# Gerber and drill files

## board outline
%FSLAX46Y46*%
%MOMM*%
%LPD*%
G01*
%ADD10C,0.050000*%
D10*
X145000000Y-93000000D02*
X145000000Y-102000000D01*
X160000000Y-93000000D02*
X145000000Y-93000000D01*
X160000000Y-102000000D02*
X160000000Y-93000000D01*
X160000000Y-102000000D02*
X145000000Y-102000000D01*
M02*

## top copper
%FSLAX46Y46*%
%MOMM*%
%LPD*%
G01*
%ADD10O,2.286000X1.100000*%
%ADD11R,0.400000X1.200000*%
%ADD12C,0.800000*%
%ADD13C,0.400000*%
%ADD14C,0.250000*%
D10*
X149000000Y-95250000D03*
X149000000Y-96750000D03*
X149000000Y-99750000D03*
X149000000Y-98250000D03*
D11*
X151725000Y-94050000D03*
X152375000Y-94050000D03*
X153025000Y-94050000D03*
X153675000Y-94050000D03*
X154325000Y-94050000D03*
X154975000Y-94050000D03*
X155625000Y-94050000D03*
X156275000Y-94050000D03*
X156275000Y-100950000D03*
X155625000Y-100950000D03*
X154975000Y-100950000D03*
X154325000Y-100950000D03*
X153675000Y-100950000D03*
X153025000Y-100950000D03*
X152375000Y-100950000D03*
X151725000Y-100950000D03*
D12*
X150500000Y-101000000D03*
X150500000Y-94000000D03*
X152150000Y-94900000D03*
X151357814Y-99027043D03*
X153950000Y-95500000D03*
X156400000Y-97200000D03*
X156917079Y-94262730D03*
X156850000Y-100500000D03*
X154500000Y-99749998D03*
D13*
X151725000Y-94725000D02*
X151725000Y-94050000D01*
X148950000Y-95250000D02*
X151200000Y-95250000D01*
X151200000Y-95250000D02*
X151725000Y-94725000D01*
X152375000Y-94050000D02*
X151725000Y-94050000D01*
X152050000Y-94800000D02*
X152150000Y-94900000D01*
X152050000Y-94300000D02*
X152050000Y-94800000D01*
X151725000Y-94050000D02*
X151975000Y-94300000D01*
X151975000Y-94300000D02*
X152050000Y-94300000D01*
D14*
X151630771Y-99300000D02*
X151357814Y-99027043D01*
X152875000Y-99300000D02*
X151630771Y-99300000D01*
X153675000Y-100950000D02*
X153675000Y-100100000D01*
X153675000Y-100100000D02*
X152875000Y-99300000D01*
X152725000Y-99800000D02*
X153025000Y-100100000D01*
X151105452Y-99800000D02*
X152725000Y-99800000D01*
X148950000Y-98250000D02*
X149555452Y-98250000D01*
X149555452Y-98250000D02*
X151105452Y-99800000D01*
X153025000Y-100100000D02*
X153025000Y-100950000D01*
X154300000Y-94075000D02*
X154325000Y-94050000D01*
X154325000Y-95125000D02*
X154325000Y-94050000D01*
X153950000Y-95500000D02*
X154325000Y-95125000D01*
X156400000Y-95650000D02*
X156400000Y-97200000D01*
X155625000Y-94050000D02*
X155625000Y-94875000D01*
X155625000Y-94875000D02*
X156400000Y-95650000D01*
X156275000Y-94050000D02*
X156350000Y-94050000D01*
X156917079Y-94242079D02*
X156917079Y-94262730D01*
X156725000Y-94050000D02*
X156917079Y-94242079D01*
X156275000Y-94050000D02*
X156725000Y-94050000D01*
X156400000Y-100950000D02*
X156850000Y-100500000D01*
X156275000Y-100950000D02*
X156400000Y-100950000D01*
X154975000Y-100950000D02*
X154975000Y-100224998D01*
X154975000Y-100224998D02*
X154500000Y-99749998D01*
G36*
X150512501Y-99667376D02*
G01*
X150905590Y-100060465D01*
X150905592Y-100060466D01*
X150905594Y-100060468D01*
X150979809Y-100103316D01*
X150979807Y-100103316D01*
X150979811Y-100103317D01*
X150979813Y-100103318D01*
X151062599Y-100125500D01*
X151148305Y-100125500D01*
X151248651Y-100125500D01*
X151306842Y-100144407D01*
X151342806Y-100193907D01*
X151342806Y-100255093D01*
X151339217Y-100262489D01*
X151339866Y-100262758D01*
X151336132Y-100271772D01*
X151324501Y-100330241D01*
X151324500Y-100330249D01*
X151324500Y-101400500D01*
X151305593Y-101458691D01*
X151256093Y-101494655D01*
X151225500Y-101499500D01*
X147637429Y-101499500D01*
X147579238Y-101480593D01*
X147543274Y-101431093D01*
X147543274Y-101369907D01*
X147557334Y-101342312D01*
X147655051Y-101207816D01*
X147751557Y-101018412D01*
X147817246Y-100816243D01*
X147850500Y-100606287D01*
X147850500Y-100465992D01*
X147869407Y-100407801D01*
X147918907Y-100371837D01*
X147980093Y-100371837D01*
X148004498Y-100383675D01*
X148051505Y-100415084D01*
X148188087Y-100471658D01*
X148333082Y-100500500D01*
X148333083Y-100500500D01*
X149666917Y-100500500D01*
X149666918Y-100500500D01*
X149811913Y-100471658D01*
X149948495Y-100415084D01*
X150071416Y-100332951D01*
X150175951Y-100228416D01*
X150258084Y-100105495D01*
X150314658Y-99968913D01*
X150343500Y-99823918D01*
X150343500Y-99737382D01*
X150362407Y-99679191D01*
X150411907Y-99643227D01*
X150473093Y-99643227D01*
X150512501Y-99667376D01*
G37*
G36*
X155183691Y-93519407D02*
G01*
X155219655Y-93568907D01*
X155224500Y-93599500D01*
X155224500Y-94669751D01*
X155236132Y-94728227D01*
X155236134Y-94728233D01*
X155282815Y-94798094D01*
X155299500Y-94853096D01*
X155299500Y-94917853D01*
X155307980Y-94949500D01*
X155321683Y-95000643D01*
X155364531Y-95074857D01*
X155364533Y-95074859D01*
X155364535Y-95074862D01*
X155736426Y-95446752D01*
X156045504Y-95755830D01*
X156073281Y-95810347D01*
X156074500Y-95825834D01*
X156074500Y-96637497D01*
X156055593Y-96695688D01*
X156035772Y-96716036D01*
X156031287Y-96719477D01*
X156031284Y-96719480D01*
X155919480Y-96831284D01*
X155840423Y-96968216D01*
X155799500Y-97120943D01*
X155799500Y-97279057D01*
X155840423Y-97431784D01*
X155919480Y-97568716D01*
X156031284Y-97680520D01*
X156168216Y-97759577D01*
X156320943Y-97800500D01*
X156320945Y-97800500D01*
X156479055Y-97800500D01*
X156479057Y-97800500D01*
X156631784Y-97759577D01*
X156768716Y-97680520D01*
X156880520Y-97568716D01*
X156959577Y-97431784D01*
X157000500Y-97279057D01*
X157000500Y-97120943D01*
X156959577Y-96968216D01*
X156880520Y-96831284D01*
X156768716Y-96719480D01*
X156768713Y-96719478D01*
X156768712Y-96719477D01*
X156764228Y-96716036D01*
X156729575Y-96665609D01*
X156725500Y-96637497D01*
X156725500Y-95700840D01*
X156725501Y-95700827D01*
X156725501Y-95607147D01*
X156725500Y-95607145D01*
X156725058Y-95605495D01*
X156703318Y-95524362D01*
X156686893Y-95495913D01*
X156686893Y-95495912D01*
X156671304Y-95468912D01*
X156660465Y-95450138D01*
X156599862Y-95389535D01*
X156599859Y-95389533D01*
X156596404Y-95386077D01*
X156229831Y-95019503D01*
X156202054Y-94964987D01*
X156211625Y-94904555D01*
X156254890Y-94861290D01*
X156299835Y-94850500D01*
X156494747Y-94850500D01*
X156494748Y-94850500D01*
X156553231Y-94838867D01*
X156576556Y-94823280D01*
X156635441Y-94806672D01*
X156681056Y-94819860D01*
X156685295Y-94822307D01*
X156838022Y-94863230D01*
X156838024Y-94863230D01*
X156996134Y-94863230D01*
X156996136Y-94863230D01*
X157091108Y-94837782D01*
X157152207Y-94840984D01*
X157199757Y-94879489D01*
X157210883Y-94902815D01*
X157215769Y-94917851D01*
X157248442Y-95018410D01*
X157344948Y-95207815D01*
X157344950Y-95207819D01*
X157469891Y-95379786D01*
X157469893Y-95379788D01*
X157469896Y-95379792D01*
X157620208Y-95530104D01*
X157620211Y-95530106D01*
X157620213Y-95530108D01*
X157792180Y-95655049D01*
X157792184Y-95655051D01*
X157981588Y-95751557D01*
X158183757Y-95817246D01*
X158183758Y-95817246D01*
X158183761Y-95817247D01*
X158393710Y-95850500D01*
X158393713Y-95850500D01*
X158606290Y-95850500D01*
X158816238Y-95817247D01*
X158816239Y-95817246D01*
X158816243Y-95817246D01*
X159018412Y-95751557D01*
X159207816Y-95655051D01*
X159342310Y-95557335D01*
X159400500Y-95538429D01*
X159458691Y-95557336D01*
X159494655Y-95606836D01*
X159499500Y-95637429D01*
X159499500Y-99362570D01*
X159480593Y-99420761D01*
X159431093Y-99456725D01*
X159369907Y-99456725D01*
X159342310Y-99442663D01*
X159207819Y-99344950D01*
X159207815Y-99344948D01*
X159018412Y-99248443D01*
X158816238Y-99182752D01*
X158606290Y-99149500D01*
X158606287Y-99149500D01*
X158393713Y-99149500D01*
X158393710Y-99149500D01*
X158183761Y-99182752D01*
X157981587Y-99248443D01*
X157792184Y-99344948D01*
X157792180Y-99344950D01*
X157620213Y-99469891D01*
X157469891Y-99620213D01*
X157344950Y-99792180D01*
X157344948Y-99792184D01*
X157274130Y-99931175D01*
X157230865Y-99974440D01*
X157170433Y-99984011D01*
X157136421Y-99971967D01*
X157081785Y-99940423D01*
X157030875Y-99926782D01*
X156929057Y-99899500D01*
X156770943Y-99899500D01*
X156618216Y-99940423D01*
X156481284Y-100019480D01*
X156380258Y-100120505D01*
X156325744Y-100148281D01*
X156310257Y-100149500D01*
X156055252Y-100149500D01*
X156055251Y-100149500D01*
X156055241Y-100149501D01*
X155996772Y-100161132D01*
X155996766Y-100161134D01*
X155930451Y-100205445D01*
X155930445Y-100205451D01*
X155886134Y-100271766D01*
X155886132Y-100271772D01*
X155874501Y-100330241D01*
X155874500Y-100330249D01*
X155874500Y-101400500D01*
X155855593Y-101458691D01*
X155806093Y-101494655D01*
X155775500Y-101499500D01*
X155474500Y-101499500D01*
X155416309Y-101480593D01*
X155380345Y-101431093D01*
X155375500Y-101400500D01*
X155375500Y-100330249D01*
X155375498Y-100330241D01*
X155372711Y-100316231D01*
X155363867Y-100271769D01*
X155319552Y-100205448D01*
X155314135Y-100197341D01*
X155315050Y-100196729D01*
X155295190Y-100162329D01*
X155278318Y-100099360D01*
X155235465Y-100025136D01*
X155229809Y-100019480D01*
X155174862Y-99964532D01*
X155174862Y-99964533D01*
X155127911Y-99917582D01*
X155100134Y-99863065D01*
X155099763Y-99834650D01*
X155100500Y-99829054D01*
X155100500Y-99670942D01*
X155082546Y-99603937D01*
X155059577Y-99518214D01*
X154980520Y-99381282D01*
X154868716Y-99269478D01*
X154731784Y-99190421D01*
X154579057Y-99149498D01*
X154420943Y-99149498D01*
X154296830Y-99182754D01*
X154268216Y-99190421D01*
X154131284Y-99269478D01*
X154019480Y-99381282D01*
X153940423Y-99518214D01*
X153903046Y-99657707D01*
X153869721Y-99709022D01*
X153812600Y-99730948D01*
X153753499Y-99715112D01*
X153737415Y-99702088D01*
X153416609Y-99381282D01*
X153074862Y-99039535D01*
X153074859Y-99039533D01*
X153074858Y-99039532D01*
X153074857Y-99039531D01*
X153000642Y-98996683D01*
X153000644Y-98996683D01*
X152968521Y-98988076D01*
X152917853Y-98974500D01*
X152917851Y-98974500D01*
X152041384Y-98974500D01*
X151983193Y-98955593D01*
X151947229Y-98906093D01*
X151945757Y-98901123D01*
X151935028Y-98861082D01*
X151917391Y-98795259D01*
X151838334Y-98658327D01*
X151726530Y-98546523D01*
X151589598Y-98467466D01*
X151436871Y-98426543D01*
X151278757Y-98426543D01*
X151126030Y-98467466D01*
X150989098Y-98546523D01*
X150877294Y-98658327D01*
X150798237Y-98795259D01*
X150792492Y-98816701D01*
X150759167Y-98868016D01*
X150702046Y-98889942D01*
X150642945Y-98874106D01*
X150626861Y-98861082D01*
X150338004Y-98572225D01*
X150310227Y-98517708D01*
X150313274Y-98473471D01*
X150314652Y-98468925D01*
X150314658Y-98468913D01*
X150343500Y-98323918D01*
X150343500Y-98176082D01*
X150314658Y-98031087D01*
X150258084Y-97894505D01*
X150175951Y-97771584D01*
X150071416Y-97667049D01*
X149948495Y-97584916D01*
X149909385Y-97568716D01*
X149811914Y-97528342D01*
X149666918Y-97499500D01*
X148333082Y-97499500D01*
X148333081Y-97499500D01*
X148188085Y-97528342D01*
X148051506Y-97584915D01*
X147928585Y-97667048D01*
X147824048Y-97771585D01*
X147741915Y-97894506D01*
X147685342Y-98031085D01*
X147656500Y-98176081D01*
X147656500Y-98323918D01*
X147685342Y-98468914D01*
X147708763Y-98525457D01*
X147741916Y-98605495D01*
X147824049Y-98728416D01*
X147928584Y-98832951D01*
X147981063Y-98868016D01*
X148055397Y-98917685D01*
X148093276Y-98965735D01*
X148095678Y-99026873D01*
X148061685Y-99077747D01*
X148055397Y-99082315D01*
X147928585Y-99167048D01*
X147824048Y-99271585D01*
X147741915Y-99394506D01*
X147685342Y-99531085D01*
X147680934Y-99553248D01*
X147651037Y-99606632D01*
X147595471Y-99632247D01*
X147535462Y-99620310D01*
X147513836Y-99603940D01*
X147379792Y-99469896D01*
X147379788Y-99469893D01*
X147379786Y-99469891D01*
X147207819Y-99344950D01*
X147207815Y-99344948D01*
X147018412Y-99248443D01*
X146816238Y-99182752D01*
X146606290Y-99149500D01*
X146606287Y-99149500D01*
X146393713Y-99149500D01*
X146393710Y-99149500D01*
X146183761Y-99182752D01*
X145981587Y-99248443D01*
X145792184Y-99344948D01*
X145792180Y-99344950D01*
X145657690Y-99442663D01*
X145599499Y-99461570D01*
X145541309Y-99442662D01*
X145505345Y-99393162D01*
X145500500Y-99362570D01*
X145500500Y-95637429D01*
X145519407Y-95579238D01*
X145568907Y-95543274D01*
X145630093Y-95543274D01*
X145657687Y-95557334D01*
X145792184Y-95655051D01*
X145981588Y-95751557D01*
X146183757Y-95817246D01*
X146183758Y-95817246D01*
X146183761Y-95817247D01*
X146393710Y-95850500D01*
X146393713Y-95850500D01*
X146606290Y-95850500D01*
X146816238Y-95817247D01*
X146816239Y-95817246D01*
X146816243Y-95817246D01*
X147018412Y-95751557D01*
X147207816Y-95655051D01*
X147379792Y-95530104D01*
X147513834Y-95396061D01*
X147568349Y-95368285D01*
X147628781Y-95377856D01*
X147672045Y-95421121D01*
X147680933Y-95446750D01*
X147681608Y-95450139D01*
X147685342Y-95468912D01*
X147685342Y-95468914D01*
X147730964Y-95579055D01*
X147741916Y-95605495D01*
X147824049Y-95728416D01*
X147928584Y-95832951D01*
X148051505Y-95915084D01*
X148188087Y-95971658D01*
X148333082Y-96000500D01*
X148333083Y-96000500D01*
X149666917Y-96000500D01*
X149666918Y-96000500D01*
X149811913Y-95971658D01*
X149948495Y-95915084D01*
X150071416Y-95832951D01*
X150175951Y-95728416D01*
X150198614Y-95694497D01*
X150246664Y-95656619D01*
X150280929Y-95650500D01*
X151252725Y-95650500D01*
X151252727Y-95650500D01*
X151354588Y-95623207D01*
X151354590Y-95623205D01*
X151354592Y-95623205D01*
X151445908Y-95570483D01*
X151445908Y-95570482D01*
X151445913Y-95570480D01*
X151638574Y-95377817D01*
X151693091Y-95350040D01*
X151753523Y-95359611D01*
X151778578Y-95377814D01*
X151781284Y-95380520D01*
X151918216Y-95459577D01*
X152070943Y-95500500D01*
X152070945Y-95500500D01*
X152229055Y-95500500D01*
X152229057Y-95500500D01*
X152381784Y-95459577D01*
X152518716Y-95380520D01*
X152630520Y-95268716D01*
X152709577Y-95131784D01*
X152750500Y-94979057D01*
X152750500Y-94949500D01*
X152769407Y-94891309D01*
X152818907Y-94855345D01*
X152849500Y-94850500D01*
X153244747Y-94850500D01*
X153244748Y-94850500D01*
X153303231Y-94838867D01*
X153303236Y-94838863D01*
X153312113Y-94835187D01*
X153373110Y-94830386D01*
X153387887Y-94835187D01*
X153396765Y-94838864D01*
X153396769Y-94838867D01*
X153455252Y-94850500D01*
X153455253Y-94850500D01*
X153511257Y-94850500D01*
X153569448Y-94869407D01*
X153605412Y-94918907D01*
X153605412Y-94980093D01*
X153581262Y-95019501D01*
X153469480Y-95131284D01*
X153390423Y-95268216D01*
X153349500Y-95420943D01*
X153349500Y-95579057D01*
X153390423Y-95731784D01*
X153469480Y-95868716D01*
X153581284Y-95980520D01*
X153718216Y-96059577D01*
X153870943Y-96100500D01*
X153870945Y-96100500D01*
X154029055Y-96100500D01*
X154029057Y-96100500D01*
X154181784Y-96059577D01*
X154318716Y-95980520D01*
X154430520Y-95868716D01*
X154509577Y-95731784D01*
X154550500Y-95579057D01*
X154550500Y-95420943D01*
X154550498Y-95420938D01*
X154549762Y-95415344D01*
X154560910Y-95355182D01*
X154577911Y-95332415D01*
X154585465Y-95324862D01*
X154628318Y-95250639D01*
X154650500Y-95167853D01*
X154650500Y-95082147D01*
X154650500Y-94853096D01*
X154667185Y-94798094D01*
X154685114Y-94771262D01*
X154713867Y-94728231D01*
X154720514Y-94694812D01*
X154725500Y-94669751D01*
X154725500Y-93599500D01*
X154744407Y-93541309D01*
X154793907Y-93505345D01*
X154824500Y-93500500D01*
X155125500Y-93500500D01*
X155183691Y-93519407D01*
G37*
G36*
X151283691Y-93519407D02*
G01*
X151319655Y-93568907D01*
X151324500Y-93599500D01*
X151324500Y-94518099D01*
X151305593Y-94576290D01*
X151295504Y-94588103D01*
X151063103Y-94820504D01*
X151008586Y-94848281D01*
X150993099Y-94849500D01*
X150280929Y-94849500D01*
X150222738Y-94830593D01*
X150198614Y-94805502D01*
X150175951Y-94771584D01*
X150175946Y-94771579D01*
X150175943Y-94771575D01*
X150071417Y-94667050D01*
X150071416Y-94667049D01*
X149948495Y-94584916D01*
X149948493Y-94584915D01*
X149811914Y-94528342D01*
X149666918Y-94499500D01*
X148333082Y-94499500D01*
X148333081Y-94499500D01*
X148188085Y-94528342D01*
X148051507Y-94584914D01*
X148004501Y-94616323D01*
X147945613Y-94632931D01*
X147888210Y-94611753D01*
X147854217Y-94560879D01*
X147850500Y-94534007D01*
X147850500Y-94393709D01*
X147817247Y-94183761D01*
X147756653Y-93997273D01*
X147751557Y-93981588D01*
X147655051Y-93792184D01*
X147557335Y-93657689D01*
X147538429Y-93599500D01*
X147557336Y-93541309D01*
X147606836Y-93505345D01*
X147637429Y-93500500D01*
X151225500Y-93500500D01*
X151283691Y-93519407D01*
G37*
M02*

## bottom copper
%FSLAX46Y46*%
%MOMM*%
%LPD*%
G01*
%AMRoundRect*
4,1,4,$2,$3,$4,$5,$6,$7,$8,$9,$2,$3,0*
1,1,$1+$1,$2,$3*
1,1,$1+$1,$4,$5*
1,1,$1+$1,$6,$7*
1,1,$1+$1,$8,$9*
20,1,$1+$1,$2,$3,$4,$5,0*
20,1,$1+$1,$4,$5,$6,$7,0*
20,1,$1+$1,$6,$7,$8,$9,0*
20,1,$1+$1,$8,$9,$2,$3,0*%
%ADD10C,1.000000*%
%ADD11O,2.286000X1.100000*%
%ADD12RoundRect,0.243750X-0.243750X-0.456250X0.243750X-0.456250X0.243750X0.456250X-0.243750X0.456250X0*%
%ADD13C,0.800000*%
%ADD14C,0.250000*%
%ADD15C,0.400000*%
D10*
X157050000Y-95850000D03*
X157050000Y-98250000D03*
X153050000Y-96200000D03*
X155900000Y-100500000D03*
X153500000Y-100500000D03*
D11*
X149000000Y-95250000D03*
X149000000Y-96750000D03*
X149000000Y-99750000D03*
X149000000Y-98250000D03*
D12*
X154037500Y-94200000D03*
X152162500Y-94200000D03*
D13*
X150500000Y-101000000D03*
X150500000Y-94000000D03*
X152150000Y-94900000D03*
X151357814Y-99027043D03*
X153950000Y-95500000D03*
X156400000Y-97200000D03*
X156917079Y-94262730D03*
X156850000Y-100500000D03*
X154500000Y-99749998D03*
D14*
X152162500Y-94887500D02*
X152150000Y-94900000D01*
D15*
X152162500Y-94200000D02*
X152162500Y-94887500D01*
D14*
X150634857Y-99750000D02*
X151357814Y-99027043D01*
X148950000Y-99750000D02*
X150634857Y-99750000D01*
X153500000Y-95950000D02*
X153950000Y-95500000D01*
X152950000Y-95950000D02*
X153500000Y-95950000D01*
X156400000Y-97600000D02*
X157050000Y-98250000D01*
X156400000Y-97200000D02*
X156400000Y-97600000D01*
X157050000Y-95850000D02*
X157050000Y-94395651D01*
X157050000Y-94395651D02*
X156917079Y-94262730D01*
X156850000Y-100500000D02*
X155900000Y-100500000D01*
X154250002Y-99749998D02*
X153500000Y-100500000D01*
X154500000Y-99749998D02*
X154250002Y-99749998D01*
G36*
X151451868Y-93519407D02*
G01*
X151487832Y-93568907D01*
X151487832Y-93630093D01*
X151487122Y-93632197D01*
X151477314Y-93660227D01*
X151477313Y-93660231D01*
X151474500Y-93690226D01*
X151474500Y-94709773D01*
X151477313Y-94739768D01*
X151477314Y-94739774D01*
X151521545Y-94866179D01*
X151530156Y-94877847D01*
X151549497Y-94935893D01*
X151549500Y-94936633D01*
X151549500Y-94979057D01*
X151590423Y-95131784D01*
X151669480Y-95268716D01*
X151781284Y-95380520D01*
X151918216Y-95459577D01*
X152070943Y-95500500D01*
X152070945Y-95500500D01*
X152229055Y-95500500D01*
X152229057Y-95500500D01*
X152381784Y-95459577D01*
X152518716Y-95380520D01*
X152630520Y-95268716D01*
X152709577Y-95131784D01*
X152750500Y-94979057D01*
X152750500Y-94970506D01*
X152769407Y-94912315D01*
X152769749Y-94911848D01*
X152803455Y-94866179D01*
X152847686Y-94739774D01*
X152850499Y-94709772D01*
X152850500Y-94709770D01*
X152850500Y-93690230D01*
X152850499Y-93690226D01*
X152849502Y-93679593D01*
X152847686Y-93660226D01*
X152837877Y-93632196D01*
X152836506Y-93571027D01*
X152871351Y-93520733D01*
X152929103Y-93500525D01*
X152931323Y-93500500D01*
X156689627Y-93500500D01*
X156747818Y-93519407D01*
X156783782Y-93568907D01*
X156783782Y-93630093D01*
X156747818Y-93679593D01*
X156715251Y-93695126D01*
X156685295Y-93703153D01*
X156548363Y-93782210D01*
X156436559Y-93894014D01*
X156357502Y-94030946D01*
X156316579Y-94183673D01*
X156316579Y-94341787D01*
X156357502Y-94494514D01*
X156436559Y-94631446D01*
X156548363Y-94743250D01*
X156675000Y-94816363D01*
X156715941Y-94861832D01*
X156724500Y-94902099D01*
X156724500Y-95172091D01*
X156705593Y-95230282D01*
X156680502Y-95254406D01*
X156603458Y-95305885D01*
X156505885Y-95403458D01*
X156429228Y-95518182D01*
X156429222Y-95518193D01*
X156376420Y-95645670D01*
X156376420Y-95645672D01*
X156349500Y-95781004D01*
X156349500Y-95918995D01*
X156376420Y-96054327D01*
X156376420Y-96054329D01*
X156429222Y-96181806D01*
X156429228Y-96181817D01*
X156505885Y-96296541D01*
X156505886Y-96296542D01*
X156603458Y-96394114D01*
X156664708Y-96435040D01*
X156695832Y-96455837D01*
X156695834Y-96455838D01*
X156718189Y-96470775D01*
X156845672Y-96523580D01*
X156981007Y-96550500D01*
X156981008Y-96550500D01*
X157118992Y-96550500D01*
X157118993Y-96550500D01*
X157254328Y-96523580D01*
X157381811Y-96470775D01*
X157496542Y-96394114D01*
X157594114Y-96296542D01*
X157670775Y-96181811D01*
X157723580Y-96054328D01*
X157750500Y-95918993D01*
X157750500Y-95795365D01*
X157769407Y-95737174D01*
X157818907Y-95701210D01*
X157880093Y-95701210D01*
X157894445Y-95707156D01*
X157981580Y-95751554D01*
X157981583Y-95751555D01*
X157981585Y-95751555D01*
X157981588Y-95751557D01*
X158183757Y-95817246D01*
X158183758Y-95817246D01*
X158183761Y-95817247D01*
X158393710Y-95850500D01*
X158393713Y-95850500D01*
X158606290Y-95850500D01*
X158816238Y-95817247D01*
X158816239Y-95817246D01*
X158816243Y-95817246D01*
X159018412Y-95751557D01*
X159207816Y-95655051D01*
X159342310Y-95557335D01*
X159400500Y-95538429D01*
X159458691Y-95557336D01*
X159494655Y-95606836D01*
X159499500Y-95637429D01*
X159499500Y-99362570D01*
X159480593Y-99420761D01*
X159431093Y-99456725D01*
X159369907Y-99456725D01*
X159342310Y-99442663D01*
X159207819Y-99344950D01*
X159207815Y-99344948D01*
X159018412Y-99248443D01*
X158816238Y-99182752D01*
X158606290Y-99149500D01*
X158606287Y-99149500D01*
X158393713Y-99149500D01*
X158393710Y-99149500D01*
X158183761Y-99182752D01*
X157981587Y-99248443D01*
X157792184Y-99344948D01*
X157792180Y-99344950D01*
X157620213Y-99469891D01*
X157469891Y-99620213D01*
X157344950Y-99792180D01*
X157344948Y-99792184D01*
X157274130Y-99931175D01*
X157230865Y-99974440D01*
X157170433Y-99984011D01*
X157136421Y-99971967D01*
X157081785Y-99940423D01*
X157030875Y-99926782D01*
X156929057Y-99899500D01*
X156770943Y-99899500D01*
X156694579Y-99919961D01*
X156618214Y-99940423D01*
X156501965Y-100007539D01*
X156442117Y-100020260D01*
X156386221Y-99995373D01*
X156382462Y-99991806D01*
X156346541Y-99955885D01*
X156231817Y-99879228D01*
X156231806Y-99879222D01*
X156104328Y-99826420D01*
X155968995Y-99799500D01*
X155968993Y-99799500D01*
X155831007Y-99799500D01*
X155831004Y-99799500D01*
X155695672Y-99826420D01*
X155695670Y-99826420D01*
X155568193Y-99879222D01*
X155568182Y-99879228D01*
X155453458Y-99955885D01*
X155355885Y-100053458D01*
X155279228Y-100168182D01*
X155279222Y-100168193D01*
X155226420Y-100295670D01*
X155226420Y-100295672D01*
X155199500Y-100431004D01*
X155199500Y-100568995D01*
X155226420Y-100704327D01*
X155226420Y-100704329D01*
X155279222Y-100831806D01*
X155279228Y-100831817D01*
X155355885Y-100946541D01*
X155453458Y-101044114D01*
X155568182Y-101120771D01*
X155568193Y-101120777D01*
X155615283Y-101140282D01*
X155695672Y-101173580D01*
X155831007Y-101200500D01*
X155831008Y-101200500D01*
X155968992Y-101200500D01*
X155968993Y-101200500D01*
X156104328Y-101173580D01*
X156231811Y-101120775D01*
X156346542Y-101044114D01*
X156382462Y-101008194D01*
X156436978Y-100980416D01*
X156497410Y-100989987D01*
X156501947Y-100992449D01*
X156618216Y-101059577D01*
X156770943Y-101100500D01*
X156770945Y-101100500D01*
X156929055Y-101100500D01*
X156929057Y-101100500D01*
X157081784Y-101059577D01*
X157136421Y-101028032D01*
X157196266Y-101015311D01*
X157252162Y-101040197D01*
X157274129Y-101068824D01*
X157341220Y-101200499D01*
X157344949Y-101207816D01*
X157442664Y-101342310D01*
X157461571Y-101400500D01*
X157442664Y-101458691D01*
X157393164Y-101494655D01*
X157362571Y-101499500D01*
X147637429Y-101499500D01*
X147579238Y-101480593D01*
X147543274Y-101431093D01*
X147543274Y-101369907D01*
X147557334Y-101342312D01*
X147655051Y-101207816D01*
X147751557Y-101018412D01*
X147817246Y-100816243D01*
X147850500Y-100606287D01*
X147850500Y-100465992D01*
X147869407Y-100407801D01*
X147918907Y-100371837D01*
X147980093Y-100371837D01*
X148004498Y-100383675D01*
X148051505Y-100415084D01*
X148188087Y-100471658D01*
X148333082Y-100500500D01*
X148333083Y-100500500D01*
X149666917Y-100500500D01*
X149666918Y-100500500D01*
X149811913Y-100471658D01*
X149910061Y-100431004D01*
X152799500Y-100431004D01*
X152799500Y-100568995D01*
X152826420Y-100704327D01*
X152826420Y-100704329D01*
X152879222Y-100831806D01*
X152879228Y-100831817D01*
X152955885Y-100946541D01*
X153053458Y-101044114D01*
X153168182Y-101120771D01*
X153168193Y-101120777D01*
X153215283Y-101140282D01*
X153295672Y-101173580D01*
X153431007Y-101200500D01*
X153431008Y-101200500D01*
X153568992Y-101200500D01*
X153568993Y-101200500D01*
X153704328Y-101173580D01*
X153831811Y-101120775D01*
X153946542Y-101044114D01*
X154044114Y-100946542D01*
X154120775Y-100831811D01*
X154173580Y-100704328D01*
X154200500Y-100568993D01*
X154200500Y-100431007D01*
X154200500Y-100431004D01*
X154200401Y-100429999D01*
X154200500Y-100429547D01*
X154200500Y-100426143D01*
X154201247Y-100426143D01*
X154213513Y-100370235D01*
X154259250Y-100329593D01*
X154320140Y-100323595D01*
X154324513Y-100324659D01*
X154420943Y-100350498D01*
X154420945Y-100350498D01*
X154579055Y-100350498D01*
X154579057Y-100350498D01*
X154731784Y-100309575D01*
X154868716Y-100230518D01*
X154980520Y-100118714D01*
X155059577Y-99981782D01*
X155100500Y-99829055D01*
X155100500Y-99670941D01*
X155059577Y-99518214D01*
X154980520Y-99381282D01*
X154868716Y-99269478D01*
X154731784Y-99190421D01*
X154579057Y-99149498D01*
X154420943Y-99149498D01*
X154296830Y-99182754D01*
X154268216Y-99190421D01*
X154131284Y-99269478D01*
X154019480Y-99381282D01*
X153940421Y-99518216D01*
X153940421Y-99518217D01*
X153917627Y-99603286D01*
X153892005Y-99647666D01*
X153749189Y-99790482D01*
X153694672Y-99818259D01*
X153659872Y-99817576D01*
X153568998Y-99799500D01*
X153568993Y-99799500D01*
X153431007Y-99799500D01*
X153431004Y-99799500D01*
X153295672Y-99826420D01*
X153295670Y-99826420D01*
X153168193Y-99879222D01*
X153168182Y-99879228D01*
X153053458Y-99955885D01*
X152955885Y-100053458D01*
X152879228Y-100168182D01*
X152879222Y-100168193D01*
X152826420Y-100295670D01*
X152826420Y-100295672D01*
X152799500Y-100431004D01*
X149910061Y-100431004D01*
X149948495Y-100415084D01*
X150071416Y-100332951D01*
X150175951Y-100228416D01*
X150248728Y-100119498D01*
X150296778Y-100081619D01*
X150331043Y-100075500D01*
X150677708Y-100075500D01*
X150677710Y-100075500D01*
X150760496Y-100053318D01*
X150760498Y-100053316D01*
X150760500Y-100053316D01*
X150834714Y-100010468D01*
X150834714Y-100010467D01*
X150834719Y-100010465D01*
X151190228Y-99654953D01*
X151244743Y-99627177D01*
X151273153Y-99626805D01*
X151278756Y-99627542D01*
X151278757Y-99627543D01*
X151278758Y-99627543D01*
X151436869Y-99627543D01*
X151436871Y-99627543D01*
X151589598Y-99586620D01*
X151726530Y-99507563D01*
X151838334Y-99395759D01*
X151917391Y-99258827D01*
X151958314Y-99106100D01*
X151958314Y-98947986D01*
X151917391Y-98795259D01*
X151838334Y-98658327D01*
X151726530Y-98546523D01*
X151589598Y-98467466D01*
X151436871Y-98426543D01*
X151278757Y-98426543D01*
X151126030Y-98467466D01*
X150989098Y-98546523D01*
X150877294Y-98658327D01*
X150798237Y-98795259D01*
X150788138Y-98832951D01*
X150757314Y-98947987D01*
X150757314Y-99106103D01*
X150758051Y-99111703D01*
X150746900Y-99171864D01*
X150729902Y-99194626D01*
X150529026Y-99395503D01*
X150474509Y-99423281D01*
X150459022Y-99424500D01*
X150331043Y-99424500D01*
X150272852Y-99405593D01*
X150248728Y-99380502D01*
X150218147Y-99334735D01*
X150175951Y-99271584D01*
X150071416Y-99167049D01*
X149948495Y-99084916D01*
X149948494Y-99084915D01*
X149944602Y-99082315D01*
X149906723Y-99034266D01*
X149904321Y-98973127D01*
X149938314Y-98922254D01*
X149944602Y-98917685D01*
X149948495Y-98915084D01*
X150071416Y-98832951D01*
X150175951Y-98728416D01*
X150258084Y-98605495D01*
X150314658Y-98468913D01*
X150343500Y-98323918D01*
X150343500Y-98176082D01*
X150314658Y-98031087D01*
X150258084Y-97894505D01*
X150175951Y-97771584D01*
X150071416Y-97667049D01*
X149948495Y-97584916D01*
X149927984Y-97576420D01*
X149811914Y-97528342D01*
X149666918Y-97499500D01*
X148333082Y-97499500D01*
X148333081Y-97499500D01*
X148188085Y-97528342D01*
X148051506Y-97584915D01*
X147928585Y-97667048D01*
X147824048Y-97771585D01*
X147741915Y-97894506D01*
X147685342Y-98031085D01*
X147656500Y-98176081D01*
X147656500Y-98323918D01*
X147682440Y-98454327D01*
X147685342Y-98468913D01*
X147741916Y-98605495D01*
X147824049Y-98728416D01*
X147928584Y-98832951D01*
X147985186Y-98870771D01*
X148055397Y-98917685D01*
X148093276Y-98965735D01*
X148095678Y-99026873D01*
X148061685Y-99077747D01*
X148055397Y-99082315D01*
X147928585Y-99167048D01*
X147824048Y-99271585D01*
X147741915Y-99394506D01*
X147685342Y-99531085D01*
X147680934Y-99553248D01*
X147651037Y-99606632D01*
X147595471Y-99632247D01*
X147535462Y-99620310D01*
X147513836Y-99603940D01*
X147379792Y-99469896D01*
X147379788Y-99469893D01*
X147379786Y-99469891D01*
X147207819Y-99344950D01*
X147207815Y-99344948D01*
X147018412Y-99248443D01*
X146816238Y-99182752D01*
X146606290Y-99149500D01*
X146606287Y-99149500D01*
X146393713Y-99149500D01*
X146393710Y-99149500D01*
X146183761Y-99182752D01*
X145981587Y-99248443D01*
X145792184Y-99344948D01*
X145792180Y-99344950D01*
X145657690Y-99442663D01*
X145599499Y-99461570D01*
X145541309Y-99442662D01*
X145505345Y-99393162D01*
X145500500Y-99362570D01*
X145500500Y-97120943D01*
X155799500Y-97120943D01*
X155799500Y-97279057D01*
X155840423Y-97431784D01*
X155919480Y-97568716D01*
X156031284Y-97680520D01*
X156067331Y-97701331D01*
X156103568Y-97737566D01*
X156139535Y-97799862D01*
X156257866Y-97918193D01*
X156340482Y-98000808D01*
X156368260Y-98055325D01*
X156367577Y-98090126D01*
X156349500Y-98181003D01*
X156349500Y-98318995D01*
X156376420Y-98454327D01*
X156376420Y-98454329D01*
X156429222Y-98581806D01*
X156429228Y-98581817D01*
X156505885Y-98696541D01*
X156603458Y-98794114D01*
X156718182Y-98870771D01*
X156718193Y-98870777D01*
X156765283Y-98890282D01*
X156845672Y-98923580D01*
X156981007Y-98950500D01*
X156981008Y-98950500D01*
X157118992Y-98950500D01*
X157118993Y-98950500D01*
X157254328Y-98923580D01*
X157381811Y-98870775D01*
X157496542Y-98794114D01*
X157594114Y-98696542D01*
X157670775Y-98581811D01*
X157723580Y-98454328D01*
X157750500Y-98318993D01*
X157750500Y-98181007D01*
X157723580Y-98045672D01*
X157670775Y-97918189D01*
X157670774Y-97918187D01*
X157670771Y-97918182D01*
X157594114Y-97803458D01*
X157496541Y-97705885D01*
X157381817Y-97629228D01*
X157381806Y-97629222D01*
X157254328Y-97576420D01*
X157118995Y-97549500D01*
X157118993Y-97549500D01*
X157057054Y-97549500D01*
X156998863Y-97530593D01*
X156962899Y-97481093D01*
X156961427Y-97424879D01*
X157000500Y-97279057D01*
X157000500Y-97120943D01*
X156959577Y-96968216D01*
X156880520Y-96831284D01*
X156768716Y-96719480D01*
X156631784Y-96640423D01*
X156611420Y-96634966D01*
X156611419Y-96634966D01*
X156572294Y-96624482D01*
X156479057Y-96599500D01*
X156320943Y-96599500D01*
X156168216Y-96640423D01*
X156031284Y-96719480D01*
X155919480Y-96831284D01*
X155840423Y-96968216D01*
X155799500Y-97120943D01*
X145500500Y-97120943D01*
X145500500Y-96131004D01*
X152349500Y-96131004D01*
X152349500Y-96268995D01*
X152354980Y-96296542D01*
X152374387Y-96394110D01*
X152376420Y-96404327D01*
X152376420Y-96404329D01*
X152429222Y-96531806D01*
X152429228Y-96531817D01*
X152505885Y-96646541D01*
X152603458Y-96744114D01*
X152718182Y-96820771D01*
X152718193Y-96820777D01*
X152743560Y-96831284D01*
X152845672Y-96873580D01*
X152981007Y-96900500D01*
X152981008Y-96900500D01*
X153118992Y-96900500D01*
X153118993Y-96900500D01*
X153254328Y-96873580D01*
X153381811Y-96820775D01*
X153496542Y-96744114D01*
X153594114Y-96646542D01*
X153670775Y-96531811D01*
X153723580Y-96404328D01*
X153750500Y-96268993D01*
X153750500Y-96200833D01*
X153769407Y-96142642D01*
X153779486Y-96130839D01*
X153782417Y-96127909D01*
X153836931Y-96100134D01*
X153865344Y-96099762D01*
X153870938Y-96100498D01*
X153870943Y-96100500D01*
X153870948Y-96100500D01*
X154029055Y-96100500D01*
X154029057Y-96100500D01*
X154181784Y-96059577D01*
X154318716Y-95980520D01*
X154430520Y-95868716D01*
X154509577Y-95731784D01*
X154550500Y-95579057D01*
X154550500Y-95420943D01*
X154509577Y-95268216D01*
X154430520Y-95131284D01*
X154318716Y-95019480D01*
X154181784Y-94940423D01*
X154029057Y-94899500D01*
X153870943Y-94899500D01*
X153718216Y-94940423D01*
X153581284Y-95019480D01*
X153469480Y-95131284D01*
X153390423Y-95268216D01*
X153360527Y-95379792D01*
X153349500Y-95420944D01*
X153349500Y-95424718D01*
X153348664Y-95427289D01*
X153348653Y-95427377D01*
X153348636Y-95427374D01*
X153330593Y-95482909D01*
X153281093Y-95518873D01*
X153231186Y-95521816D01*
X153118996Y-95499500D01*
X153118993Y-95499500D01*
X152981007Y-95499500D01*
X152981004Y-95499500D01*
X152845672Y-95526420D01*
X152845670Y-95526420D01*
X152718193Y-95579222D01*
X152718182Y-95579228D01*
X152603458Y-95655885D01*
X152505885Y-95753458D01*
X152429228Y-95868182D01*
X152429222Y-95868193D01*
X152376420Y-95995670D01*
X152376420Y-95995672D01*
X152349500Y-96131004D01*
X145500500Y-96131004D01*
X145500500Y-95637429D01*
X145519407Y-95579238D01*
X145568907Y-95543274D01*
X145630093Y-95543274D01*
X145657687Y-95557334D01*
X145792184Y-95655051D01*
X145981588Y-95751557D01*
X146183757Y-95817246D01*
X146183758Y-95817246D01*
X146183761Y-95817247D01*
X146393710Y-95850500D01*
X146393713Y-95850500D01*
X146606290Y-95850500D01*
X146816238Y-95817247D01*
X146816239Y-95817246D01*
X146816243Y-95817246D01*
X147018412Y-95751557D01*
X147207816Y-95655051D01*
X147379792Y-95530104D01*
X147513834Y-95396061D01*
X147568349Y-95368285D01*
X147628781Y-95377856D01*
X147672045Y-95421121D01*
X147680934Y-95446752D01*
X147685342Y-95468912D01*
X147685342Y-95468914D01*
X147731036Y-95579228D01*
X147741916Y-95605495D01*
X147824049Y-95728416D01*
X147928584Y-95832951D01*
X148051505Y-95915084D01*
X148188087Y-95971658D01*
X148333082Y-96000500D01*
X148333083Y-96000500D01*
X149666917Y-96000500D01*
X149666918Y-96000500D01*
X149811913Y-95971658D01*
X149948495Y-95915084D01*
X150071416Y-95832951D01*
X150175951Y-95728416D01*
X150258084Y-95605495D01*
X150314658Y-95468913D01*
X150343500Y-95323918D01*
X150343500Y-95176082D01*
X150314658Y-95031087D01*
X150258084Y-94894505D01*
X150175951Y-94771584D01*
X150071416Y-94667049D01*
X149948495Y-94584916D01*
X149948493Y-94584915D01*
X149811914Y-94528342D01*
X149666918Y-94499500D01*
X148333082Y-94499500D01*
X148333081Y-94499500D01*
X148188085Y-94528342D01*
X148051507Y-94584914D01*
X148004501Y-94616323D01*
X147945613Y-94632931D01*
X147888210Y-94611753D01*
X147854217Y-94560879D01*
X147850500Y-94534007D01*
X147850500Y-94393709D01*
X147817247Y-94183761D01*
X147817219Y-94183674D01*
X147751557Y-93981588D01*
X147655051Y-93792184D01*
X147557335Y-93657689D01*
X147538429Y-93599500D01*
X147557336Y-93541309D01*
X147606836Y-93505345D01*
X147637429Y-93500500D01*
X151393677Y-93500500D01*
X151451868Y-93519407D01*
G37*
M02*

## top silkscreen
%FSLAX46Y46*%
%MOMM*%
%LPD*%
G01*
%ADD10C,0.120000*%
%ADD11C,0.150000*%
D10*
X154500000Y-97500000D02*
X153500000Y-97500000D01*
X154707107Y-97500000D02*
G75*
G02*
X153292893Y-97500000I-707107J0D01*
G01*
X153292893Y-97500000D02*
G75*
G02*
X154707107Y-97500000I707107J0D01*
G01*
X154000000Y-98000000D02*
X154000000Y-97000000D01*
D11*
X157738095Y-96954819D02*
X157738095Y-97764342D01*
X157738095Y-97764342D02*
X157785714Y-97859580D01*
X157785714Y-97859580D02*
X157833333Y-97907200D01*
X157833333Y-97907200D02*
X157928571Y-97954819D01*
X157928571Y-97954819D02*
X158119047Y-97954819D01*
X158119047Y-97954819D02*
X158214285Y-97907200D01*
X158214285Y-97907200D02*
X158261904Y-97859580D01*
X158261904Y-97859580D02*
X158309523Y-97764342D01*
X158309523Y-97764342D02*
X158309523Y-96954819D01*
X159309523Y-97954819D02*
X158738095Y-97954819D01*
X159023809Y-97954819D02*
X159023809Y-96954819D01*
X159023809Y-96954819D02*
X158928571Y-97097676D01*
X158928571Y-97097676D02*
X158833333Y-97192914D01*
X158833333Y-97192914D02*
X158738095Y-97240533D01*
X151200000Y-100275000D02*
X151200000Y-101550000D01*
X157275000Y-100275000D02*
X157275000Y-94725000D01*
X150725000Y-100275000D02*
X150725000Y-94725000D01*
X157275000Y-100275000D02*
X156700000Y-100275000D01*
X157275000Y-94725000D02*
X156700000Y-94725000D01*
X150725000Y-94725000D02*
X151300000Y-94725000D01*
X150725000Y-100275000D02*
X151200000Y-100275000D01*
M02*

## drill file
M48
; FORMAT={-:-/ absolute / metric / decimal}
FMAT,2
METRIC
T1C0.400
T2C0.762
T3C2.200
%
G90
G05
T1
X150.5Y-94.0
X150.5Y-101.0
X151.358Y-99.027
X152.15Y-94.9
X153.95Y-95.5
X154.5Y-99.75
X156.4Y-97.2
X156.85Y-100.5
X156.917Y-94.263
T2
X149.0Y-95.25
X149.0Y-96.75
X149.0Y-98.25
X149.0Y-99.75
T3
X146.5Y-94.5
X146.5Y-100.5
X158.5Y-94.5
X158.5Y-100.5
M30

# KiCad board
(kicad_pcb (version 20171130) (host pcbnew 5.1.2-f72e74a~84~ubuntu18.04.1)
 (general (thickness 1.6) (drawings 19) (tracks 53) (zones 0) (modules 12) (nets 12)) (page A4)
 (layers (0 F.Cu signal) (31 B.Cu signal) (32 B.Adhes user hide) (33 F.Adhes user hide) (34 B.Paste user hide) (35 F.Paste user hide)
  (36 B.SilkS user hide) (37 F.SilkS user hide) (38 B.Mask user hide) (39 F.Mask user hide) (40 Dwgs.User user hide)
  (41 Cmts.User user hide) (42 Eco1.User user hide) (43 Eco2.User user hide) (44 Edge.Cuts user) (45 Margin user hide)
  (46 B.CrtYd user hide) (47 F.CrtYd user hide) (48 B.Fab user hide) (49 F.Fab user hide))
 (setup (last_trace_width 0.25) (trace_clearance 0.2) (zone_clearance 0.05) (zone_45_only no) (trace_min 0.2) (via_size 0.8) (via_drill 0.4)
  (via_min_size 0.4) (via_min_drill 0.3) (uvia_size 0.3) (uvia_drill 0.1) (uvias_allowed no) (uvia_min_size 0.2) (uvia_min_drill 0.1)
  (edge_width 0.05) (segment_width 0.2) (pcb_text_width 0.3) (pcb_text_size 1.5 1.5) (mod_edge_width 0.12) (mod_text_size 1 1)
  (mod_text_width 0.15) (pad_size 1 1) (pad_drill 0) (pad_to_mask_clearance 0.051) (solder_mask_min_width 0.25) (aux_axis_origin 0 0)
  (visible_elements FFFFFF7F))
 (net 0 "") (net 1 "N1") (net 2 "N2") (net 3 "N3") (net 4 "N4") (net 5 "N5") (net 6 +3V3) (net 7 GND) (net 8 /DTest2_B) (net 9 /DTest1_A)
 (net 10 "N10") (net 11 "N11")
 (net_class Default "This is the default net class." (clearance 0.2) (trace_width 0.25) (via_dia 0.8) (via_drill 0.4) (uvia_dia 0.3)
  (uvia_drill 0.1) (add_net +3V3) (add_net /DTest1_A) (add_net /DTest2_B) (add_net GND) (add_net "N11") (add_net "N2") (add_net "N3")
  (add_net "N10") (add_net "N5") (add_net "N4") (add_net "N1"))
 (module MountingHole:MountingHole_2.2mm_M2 (layer F.Cu) (at 146.5 100.5)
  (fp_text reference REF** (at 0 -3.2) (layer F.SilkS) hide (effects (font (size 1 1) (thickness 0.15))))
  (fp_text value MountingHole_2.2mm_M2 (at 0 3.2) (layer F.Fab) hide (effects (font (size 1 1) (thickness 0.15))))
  (pad 1 np_thru_hole circle (at 0 0) (size 2.2 2.2) (drill 2.2) (layers *.Cu *.Mask)))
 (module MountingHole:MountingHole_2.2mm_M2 (layer F.Cu) (at 146.5 94.5)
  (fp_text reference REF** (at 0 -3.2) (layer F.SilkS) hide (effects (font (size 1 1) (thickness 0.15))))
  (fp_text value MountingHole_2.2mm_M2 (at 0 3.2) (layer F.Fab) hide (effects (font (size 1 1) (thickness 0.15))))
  (pad 1 np_thru_hole circle (at 0 0) (size 2.2 2.2) (drill 2.2) (layers *.Cu *.Mask)))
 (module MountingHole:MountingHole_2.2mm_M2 (layer F.Cu) (at 158.5 94.5)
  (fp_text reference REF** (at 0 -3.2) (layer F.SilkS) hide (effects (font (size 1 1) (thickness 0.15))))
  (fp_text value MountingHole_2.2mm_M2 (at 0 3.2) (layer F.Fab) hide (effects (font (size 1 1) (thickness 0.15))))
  (pad 1 np_thru_hole circle (at 0 0) (size 2.2 2.2) (drill 2.2) (layers *.Cu *.Mask)))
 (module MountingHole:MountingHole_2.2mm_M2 (layer F.Cu) (at 158.5 100.5)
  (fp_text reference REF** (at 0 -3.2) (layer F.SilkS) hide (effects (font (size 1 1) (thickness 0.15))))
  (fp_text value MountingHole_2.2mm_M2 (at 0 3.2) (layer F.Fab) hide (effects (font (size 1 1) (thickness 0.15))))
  (pad 1 np_thru_hole circle (at 0 0) (size 2.2 2.2) (drill 2.2) (layers *.Cu *.Mask)))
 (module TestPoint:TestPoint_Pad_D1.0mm (layer B.Cu) (at 157.05 95.85)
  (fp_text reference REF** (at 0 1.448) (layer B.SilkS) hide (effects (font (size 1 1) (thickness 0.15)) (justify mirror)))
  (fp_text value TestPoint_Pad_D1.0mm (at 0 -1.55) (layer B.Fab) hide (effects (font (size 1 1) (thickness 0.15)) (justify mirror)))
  (pad 1 smd circle (at 0 0) (size 1 1) (layers B.Cu B.Mask) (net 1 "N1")))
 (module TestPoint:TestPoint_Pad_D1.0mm (layer B.Cu) (at 157.05 98.25)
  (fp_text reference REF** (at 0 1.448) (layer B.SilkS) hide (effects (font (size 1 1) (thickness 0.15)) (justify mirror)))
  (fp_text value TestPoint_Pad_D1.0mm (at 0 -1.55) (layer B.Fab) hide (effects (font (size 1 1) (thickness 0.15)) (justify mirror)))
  (pad 1 smd circle (at 0 0) (size 1 1) (layers B.Cu B.Mask) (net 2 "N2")))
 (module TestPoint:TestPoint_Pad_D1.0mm (layer B.Cu) (at 153.05 96.2)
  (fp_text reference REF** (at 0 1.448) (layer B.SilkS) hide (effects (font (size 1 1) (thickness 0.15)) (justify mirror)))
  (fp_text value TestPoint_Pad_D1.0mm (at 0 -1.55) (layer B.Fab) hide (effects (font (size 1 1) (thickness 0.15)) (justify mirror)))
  (pad 1 smd circle (at 0 0) (size 1 1) (layers B.Cu B.Mask) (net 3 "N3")))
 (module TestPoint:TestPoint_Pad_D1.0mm (layer B.Cu) (at 155.9 100.5)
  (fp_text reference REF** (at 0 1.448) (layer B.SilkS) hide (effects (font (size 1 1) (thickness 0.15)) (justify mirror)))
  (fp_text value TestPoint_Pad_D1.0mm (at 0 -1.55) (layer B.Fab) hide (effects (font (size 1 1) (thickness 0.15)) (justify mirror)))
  (pad 1 smd circle (at 0 0) (size 1 1) (layers B.Cu B.Mask) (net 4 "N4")))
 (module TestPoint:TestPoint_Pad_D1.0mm (layer B.Cu) (at 153.5 100.5)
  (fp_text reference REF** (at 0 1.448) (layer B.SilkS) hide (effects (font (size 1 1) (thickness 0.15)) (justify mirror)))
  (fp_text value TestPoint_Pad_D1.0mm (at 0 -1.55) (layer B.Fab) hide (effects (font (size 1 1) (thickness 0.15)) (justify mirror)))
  (pad 1 smd circle (at 0 0) (size 1 1) (layers B.Cu B.Mask) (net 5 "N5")))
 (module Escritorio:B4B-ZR (layer B.Cu) (at 149.45 97.5 270)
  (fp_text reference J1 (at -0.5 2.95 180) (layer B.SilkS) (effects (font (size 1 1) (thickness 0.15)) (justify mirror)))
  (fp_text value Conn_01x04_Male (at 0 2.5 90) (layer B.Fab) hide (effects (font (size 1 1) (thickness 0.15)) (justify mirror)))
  (pad 1 thru_hole oval (at -2.25 0.45 270) (size 1.1 2.286) (drill 0.762) (layers *.Cu *.Mask) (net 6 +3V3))
  (pad 2 thru_hole oval (at -0.75 0.45 270) (size 1.1 2.286) (drill 0.762) (layers *.Cu *.Mask) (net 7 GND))
  (pad 4 thru_hole oval (at 2.25 0.45 270) (size 1.1 2.286) (drill 0.762) (layers *.Cu *.Mask) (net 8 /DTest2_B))
  (pad 3 thru_hole oval (at 0.75 0.45 270) (size 1.1 2.286) (drill 0.762) (layers *.Cu *.Mask) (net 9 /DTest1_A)))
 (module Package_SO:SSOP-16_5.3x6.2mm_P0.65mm (layer F.Cu) (at 154 97.5 90)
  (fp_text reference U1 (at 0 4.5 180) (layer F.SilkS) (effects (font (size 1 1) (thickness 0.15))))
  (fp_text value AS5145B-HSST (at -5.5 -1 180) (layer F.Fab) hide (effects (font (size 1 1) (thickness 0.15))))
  (fp_line (start -2.775 -2.8) (end -4.05 -2.8) (layer F.SilkS) (width 0.15))
  (fp_line (start -2.775 3.275) (end 2.775 3.275) (layer F.SilkS) (width 0.15))
  (fp_line (start -2.775 -3.275) (end 2.775 -3.275) (layer F.SilkS) (width 0.15))
  (fp_line (start -2.775 3.275) (end -2.775 2.7) (layer F.SilkS) (width 0.15))
  (fp_line (start 2.775 3.275) (end 2.775 2.7) (layer F.SilkS) (width 0.15))
  (fp_line (start 2.775 -3.275) (end 2.775 -2.7) (layer F.SilkS) (width 0.15))
  (fp_line (start -2.775 -3.275) (end -2.775 -2.8) (layer F.SilkS) (width 0.15))
  (pad 16 smd rect (at 3.45 -2.275 90) (size 1.2 0.4) (layers F.Cu F.Paste F.Mask) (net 6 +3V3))
  (pad 15 smd rect (at 3.45 -1.625 90) (size 1.2 0.4) (layers F.Cu F.Paste F.Mask) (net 6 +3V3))
  (pad 14 smd rect (at 3.45 -0.975 90) (size 1.2 0.4) (layers F.Cu F.Paste F.Mask))
  (pad 13 smd rect (at 3.45 -0.325 90) (size 1.2 0.4) (layers F.Cu F.Paste F.Mask))
  (pad 12 smd rect (at 3.45 0.325 90) (size 1.2 0.4) (layers F.Cu F.Paste F.Mask) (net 3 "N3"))
  (pad 11 smd rect (at 3.45 0.975 90) (size 1.2 0.4) (layers F.Cu F.Paste F.Mask) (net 7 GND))
  (pad 10 smd rect (at 3.45 1.625 90) (size 1.2 0.4) (layers F.Cu F.Paste F.Mask) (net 2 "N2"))
  (pad 9 smd rect (at 3.45 2.275 90) (size 1.2 0.4) (layers F.Cu F.Paste F.Mask) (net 1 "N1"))
  (pad 8 smd rect (at -3.45 2.275 90) (size 1.2 0.4) (layers F.Cu F.Paste F.Mask) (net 4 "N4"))
  (pad 7 smd rect (at -3.45 1.625 90) (size 1.2 0.4) (layers F.Cu F.Paste F.Mask) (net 7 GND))
  (pad 6 smd rect (at -3.45 0.975 90) (size 1.2 0.4) (layers F.Cu F.Paste F.Mask) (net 5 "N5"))
  (pad 5 smd rect (at -3.45 0.325 90) (size 1.2 0.4) (layers F.Cu F.Paste F.Mask))
  (pad 4 smd rect (at -3.45 -0.325 90) (size 1.2 0.4) (layers F.Cu F.Paste F.Mask) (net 8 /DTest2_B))
  (pad 3 smd rect (at -3.45 -0.975 90) (size 1.2 0.4) (layers F.Cu F.Paste F.Mask) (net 9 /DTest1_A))
  (pad 2 smd rect (at -3.45 -1.625 90) (size 1.2 0.4) (layers F.Cu F.Paste F.Mask) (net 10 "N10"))
  (pad 1 smd rect (at -3.45 -2.275 90) (size 1.2 0.4) (layers F.Cu F.Paste F.Mask) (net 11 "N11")))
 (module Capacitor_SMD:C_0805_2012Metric (layer B.Cu) (at 153.1 94.2)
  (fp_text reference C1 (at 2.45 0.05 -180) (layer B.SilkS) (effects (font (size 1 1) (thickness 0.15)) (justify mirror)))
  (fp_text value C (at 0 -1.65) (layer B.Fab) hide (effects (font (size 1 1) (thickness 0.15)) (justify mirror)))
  (pad 2 smd roundrect (at 0.9375 0) (size 0.975 1.4) (layers B.Cu B.Paste B.Mask) (roundrect_rratio 0.25) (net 7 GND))
  (pad 1 smd roundrect (at -0.9375 0) (size 0.975 1.4) (layers B.Cu B.Paste B.Mask) (roundrect_rratio 0.25) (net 6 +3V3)))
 (gr_line (start 154.5 97.5) (end 153.5 97.5) (layer F.SilkS) (width 0.12))
 (gr_circle (center 154 97.5) (end 153.5 98) (layer F.SilkS) (width 0.12))
 (gr_line (start 154 98) (end 154 97) (layer F.SilkS) (width 0.12))
 (gr_line (start 145 93) (end 145 102) (layer Edge.Cuts) (width 0.05))
 (gr_line (start 160 93) (end 145 93) (layer Edge.Cuts) (width 0.05))
 (gr_line (start 160 102) (end 160 93) (layer Edge.Cuts) (width 0.05))
 (gr_line (start 160 102) (end 145 102) (layer Edge.Cuts) (width 0.05))
 (via (at 150.5 101) (size 0.8) (drill 0.4) (layers F.Cu B.Cu) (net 7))
 (via (at 150.5 94) (size 0.8) (drill 0.4) (layers F.Cu B.Cu) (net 7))
 (segment (start 151.725 94.725) (end 151.725 94.05) (width 0.4) (layer F.Cu) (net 6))
 (segment (start 148.95 95.25) (end 151.2 95.25) (width 0.4) (layer F.Cu) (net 6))
 (segment (start 151.2 95.25) (end 151.725 94.725) (width 0.4) (layer F.Cu) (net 6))
 (via (at 152.15 94.9) (size 0.8) (drill 0.4) (layers F.Cu B.Cu) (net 6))
 (segment (start 152.1625 94.8875) (end 152.15 94.9) (width 0.25) (layer B.Cu) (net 6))
 (segment (start 152.1625 94.2) (end 152.1625 94.8875) (width 0.4) (layer B.Cu) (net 6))
 (segment (start 152.375 94.05) (end 151.725 94.05) (width 0.4) (layer F.Cu) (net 6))
 (segment (start 152.05 94.8) (end 152.15 94.9) (width 0.4) (layer F.Cu) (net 6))
 (segment (start 152.05 94.3) (end 152.05 94.8) (width 0.4) (layer F.Cu) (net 6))
 (segment (start 151.725 94.05) (end 151.975 94.3) (width 0.4) (layer F.Cu) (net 6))
 (segment (start 151.975 94.3) (end 152.05 94.3) (width 0.4) (layer F.Cu) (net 6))
 (via (at 151.357814 99.027043) (size 0.8) (drill 0.4) (layers F.Cu B.Cu) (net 8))
 (segment (start 150.634857 99.75) (end 151.357814 99.027043) (width 0.25) (layer B.Cu) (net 8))
 (segment (start 148.95 99.75) (end 150.634857 99.75) (width 0.25) (layer B.Cu) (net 8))
 (segment (start 151.630771 99.3) (end 151.357814 99.027043) (width 0.25) (layer F.Cu) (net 8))
 (segment (start 152.875 99.3) (end 151.630771 99.3) (width 0.25) (layer F.Cu) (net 8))
 (segment (start 153.675 100.95) (end 153.675 100.1) (width 0.25) (layer F.Cu) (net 8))
 (segment (start 153.675 100.1) (end 152.875 99.3) (width 0.25) (layer F.Cu) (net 8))
 (segment (start 152.725 99.8) (end 153.025 100.1) (width 0.25) (layer F.Cu) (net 9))
 (segment (start 151.105452 99.8) (end 152.725 99.8) (width 0.25) (layer F.Cu) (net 9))
 (segment (start 148.95 98.25) (end 149.555452 98.25) (width 0.25) (layer F.Cu) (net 9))
 (segment (start 149.555452 98.25) (end 151.105452 99.8) (width 0.25) (layer F.Cu) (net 9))
 (segment (start 153.025 100.1) (end 153.025 100.95) (width 0.25) (layer F.Cu) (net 9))
 (via (at 153.95 95.5) (size 0.8) (drill 0.4) (layers F.Cu B.Cu) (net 3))
 (segment (start 154.3 94.075) (end 154.325 94.05) (width 0.25) (layer F.Cu) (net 3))
 (segment (start 153.5 95.95) (end 153.95 95.5) (width 0.25) (layer B.Cu) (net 3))
 (segment (start 152.95 95.95) (end 153.5 95.95) (width 0.25) (layer B.Cu) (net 3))
 (segment (start 154.325 95.125) (end 154.325 94.05) (width 0.25) (layer F.Cu) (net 3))
 (segment (start 153.95 95.5) (end 154.325 95.125) (width 0.25) (layer F.Cu) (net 3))
 (segment (start 156.4 97.6) (end 157.05 98.25) (width 0.25) (layer B.Cu) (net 2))
 (via (at 156.4 97.2) (size 0.8) (drill 0.4) (layers F.Cu B.Cu) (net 2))
 (segment (start 156.4 97.2) (end 156.4 97.6) (width 0.25) (layer B.Cu) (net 2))
 (segment (start 156.4 95.65) (end 156.4 97.2) (width 0.25) (layer F.Cu) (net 2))
 (segment (start 155.625 94.05) (end 155.625 94.875) (width 0.25) (layer F.Cu) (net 2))
 (segment (start 155.625 94.875) (end 156.4 95.65) (width 0.25) (layer F.Cu) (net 2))
 (segment (start 156.275 94.05) (end 156.35 94.05) (width 0.25) (layer F.Cu) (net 1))
 (segment (start 157.05 95.85) (end 157.05 94.395651) (width 0.25) (layer B.Cu) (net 1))
 (segment (start 156.917079 94.242079) (end 156.917079 94.26273) (width 0.25) (layer F.Cu) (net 1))
 (segment (start 156.725 94.05) (end 156.917079 94.242079) (width 0.25) (layer F.Cu) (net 1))
 (via (at 156.917079 94.26273) (size 0.8) (drill 0.4) (layers F.Cu B.Cu) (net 1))
 (segment (start 157.05 94.395651) (end 156.917079 94.26273) (width 0.25) (layer B.Cu) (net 1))
 (segment (start 156.275 94.05) (end 156.725 94.05) (width 0.25) (layer F.Cu) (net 1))
 (via (at 156.85 100.5) (size 0.8) (drill 0.4) (layers F.Cu B.Cu) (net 4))
 (segment (start 156.4 100.95) (end 156.85 100.5) (width 0.25) (layer F.Cu) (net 4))
 (segment (start 156.275 100.95) (end 156.4 100.95) (width 0.25) (layer F.Cu) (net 4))
 (segment (start 156.85 100.5) (end 155.9 100.5) (width 0.25) (layer B.Cu) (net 4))
 (segment (start 154.975 100.95) (end 154.975 100.224998) (width 0.25) (layer F.Cu) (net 5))
 (via (at 154.5 99.749998) (size 0.8) (drill 0.4) (layers F.Cu B.Cu) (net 5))
 (segment (start 154.975 100.224998) (end 154.5 99.749998) (width 0.25) (layer F.Cu) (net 5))
 (segment (start 154.250002 99.749998) (end 153.5 100.5) (width 0.25) (layer B.Cu) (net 5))
 (segment (start 154.5 99.749998) (end 154.250002 99.749998) (width 0.25) (layer B.Cu) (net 5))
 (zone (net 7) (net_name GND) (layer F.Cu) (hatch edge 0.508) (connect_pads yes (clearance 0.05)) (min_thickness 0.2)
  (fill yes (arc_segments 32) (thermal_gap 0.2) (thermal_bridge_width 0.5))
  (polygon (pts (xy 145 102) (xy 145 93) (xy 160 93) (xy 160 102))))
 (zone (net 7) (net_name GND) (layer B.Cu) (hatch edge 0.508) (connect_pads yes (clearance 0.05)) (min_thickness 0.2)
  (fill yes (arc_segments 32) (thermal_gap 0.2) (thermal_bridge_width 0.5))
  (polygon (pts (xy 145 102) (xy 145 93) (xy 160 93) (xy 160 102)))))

